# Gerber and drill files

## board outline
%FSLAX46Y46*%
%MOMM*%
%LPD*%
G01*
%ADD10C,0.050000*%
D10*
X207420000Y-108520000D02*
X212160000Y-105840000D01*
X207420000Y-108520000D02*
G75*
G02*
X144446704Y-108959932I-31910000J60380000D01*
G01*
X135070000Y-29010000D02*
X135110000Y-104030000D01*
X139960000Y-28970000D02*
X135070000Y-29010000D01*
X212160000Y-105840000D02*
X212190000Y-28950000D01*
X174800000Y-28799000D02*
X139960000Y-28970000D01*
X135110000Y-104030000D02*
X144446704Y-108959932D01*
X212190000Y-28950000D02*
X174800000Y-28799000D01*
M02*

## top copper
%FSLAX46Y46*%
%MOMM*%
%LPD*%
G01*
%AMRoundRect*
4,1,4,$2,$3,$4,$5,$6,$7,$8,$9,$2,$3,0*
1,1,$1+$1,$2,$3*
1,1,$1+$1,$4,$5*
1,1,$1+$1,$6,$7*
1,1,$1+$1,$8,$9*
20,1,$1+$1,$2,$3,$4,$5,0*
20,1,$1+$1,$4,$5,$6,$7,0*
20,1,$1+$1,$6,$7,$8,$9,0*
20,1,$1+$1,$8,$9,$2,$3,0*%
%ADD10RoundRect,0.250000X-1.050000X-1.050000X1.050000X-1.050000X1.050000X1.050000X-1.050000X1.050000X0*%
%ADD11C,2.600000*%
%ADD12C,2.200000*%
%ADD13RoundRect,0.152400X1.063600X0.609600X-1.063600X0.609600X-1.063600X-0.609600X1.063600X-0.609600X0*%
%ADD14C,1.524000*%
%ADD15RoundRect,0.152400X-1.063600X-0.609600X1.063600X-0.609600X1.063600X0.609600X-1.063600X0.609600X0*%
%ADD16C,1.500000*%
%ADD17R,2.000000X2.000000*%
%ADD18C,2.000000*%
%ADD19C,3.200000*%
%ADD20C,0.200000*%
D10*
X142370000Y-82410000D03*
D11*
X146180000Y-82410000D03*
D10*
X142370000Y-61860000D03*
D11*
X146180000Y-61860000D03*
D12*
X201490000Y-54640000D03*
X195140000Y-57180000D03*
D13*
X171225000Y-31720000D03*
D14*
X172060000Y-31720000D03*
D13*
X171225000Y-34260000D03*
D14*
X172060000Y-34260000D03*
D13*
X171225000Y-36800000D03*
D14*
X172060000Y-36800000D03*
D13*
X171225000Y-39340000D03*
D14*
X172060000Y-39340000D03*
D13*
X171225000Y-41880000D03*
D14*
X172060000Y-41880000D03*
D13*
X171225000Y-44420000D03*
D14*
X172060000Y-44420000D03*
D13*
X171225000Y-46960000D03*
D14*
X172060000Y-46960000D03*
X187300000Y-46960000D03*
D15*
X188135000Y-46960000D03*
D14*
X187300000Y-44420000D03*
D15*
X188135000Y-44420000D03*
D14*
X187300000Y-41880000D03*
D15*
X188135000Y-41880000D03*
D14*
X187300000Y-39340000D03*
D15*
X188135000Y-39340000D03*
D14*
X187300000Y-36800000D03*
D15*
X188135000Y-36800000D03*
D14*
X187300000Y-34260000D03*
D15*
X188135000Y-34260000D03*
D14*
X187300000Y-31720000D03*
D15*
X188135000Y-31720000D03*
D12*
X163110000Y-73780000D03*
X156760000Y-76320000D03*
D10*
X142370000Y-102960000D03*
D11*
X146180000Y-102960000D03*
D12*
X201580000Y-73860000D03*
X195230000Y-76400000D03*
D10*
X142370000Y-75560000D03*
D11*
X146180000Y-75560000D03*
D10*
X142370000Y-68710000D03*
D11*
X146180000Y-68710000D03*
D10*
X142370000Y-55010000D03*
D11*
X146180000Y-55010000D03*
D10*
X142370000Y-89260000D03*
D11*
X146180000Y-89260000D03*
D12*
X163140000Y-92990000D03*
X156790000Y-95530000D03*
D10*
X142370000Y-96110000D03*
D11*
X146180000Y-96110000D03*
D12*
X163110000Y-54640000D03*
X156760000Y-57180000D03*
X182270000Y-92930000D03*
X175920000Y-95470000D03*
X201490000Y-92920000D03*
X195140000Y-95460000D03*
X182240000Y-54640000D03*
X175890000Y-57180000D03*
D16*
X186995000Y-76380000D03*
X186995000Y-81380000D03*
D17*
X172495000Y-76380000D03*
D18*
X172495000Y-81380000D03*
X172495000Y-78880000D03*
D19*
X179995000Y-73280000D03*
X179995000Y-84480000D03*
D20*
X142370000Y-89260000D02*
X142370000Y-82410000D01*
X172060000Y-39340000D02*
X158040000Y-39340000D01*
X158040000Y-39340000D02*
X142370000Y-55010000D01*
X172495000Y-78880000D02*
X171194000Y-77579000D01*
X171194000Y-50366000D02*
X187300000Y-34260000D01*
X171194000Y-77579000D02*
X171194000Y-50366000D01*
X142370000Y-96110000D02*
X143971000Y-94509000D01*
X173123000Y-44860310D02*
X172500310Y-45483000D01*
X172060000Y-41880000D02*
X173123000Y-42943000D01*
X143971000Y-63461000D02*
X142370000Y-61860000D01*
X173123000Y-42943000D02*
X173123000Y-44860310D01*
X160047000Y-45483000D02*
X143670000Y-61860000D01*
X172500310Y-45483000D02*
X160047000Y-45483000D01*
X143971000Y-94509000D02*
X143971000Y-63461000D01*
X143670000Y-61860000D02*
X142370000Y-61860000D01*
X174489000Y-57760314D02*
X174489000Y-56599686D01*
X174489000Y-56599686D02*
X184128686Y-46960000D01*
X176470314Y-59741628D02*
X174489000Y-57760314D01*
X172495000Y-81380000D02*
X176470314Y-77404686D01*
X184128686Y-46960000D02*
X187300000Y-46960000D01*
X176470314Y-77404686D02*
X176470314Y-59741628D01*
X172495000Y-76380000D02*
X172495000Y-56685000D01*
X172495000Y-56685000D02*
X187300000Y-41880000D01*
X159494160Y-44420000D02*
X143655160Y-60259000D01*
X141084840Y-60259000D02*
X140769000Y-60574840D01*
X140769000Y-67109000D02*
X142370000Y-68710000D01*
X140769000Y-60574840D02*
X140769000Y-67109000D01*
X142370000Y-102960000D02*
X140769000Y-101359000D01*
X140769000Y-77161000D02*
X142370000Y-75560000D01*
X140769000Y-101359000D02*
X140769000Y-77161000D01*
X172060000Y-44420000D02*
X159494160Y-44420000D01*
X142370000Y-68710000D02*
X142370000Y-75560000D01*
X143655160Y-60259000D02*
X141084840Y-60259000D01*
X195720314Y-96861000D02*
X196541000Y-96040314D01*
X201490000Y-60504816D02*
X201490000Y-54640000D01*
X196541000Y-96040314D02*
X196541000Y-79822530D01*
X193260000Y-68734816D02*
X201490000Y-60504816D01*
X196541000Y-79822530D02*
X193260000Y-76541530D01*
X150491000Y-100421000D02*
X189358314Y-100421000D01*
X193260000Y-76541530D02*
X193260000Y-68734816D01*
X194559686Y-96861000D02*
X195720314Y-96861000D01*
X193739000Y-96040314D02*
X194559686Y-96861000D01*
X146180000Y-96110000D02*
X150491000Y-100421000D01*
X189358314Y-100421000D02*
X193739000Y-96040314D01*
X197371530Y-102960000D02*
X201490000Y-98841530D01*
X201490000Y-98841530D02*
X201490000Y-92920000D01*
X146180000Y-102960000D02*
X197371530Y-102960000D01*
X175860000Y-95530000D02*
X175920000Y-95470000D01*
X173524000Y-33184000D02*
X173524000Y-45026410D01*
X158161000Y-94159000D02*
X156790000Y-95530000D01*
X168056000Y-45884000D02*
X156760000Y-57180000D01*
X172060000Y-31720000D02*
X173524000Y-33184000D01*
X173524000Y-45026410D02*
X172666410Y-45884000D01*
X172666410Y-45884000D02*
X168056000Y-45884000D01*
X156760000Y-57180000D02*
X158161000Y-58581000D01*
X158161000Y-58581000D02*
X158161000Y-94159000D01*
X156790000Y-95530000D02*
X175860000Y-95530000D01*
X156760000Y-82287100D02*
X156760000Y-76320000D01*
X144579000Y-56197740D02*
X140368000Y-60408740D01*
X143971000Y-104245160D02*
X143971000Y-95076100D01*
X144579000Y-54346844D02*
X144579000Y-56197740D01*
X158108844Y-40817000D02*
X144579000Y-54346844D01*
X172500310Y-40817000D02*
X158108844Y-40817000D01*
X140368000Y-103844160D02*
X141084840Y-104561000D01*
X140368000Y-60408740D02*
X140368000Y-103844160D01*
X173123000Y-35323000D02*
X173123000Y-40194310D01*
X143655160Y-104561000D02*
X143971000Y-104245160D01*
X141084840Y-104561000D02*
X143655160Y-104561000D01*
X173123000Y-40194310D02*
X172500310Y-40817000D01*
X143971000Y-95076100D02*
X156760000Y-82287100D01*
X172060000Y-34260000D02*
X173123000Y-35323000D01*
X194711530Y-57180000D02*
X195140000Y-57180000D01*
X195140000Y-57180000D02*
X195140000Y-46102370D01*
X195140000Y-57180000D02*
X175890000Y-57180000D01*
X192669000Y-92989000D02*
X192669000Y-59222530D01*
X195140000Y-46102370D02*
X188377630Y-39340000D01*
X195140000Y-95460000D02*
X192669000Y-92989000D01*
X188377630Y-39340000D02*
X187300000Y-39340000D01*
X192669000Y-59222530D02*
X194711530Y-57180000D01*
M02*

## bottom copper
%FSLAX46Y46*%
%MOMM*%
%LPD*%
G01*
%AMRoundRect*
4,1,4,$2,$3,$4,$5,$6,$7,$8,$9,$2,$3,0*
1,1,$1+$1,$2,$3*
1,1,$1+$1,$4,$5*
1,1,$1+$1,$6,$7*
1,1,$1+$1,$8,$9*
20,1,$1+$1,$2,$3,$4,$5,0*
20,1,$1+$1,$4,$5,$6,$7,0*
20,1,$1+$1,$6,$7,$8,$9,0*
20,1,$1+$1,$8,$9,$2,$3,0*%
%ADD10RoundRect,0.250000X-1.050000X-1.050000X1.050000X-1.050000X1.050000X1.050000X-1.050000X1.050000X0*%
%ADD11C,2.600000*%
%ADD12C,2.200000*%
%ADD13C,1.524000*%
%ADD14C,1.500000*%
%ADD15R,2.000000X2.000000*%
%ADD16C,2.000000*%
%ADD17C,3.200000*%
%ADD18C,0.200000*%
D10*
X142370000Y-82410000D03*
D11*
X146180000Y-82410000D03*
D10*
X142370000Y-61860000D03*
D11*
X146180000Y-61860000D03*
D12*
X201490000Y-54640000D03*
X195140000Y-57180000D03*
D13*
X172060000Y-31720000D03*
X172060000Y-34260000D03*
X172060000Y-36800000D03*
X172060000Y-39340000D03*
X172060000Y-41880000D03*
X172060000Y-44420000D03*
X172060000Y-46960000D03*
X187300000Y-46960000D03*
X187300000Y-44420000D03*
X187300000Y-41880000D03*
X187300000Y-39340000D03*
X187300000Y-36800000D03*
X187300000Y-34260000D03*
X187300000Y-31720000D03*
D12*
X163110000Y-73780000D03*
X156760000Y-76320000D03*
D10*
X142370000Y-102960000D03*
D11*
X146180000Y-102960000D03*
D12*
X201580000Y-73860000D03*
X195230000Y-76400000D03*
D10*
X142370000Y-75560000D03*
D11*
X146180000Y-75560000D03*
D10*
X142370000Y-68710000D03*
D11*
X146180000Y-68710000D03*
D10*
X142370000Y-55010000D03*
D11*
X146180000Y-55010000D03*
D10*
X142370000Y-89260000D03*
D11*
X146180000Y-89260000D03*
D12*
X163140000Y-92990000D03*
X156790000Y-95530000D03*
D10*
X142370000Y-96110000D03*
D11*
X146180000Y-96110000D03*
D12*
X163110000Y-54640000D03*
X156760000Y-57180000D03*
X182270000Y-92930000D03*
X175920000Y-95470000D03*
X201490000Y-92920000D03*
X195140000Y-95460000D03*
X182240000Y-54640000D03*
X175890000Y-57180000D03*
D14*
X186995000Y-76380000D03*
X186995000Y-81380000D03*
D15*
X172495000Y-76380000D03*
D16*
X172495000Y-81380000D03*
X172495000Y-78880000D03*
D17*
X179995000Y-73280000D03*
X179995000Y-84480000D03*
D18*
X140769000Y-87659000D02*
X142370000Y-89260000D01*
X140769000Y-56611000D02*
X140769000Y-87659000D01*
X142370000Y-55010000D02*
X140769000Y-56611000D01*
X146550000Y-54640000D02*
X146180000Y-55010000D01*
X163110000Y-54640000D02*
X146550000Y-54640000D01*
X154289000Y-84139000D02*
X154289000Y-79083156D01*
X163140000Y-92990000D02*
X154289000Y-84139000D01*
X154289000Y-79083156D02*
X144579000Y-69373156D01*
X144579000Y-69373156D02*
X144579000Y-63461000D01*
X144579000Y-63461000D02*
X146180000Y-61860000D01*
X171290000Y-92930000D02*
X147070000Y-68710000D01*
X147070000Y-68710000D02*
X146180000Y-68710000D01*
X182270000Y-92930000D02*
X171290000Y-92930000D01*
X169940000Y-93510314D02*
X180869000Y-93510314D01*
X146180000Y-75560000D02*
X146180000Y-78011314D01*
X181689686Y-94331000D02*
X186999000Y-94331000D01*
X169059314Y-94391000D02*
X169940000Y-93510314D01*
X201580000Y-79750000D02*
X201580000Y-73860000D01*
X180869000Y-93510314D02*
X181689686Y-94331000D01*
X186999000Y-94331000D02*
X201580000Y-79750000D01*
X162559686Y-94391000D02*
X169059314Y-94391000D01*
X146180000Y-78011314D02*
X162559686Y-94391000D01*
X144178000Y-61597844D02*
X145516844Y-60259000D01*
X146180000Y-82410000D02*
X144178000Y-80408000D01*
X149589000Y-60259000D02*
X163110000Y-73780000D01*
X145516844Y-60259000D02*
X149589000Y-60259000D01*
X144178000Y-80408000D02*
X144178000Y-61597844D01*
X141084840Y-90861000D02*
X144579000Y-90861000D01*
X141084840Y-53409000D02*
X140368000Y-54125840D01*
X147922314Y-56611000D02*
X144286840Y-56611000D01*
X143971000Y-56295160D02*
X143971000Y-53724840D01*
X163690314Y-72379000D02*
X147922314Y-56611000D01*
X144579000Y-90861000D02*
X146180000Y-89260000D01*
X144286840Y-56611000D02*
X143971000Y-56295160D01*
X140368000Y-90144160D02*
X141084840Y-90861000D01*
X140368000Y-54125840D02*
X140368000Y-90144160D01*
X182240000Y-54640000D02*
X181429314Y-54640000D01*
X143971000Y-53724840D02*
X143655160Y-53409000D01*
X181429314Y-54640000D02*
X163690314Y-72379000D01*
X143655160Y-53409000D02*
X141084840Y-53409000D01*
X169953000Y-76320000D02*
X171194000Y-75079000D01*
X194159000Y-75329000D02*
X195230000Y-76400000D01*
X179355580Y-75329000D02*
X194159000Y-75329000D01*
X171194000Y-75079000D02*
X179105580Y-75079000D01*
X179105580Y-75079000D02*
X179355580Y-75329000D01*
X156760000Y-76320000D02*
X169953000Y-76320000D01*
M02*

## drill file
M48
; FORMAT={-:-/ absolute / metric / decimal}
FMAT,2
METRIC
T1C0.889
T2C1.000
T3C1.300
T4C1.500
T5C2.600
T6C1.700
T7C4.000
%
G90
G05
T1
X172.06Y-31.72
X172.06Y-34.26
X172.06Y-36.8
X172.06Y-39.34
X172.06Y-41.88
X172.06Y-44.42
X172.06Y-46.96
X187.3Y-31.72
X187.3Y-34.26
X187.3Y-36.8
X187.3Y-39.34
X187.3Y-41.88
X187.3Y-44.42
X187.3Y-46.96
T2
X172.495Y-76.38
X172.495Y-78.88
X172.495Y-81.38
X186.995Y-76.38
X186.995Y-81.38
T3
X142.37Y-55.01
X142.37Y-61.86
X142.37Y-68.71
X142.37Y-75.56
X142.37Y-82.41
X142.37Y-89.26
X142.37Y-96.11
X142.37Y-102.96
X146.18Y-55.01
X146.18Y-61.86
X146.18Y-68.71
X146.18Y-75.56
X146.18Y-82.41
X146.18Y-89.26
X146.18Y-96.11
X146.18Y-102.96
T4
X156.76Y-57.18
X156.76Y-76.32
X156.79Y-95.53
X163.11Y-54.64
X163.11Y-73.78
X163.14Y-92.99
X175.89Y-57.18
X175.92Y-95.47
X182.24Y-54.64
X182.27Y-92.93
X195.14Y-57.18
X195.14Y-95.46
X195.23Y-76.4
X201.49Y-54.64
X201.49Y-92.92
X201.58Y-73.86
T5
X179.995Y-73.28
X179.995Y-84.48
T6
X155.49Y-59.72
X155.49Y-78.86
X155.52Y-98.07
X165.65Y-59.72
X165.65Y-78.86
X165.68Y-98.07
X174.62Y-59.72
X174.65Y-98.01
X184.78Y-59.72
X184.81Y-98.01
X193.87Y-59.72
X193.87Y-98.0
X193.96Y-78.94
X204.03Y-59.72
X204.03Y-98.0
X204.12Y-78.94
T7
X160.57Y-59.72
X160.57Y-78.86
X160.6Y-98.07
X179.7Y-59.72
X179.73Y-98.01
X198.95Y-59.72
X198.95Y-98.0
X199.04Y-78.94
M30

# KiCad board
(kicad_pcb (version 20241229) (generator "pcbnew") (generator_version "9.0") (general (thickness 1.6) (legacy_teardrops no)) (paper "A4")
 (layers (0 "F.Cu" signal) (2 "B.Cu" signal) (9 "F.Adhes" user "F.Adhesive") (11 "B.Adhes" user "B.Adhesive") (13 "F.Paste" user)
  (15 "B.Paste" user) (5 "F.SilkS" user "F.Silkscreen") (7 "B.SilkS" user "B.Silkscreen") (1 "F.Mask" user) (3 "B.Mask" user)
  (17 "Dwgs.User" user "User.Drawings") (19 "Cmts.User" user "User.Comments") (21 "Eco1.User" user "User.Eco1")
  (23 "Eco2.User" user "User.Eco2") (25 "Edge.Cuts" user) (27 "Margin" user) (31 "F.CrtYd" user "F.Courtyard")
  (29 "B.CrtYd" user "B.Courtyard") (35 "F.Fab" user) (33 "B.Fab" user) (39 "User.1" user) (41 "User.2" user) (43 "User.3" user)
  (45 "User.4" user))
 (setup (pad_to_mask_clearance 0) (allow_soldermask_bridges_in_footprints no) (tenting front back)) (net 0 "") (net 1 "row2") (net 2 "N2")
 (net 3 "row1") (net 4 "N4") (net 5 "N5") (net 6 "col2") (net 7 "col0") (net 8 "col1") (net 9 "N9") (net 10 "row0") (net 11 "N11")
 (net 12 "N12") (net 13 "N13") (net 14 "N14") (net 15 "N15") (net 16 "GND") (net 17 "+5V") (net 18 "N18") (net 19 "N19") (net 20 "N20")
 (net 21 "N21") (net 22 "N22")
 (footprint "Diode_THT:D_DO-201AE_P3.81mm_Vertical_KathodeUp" (layer "F.Cu") (at 142.37 82.41)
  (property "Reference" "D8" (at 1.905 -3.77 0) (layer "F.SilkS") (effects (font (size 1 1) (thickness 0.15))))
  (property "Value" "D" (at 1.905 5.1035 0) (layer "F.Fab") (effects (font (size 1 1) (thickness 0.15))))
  (pad "1" thru_hole roundrect (at 0 0) (size 2.6 2.6) (drill 1.3) (layers "*.Cu" "*.Mask") (remove_unused_layers no)
   (roundrect_rratio 0.096154) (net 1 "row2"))
  (pad "2" thru_hole circle (at 3.81 0) (size 2.6 2.6) (drill 1.3) (layers "*.Cu" "*.Mask") (remove_unused_layers no) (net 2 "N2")))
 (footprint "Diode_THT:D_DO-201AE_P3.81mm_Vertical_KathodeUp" (layer "F.Cu") (at 142.37 61.86)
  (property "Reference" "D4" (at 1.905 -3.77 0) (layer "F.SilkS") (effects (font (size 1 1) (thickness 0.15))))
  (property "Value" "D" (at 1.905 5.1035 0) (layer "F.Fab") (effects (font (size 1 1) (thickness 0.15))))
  (pad "1" thru_hole roundrect (at 0 0) (size 2.6 2.6) (drill 1.3) (layers "*.Cu" "*.Mask") (remove_unused_layers no)
   (roundrect_rratio 0.096154) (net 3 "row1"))
  (pad "2" thru_hole circle (at 3.81 0) (size 2.6 2.6) (drill 1.3) (layers "*.Cu" "*.Mask") (remove_unused_layers no) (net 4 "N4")))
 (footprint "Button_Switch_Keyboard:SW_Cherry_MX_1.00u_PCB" (layer "F.Cu") (at 201.49 54.64)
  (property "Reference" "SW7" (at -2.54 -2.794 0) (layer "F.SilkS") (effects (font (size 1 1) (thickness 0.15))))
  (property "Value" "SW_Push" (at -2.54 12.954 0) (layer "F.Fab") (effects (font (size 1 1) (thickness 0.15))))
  (pad "" np_thru_hole circle (at -7.62 5.08) (size 1.7 1.7) (drill 1.7) (layers "*.Cu" "*.Mask"))
  (pad "" np_thru_hole circle (at -2.54 5.08) (size 4 4) (drill 4) (layers "*.Cu" "*.Mask"))
  (pad "" np_thru_hole circle (at 2.54 5.08) (size 1.7 1.7) (drill 1.7) (layers "*.Cu" "*.Mask"))
  (pad "1" thru_hole circle (at 0 0) (size 2.2 2.2) (drill 1.5) (layers "*.Cu" "*.Mask") (remove_unused_layers no) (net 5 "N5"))
  (pad "2" thru_hole circle (at -6.35 2.54) (size 2.2 2.2) (drill 1.5) (layers "*.Cu" "*.Mask") (remove_unused_layers no) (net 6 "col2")))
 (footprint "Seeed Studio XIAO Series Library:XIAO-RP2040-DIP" (layer "F.Cu") (at 179.68 39.34)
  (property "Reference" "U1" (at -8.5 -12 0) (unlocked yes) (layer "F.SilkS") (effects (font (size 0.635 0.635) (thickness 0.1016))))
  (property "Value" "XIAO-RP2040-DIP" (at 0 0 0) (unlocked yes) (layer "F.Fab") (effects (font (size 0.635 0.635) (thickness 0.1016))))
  (pad "1" smd roundrect (at -8.455 -7.62 180) (size 2.432 1.524) (layers "F.Cu" "F.Mask") (roundrect_rratio 0.1) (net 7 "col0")
   (thermal_bridge_angle 45))
  (pad "1" thru_hole circle (at -7.62 -7.62 180) (size 1.524 1.524) (drill 0.889) (layers "*.Cu" "*.Mask") (remove_unused_layers no)
   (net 7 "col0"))
  (pad "2" smd roundrect (at -8.455 -5.08 180) (size 2.432 1.524) (layers "F.Cu" "F.Mask") (roundrect_rratio 0.1) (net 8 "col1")
   (thermal_bridge_angle 45))
  (pad "2" thru_hole circle (at -7.62 -5.08 180) (size 1.524 1.524) (drill 0.889) (layers "*.Cu" "*.Mask") (remove_unused_layers no)
   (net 8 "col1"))
  (pad "3" smd roundrect (at -8.455 -2.54 180) (size 2.432 1.524) (layers "F.Cu" "F.Mask") (roundrect_rratio 0.1) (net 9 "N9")
   (thermal_bridge_angle 45))
  (pad "3" thru_hole circle (at -7.62 -2.54 180) (size 1.524 1.524) (drill 0.889) (layers "*.Cu" "*.Mask") (remove_unused_layers no)
   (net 9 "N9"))
  (pad "4" smd roundrect (at -8.455 0 180) (size 2.432 1.524) (layers "F.Cu" "F.Mask") (roundrect_rratio 0.1) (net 1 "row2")
   (thermal_bridge_angle 45))
  (pad "4" thru_hole circle (at -7.62 0 180) (size 1.524 1.524) (drill 0.889) (layers "*.Cu" "*.Mask") (remove_unused_layers no)
   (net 1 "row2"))
  (pad "5" smd roundrect (at -8.455 2.54 180) (size 2.432 1.524) (layers "F.Cu" "F.Mask") (roundrect_rratio 0.1) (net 3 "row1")
   (thermal_bridge_angle 45))
  (pad "5" thru_hole circle (at -7.62 2.54 180) (size 1.524 1.524) (drill 0.889) (layers "*.Cu" "*.Mask") (remove_unused_layers no)
   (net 3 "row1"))
  (pad "6" smd roundrect (at -8.455 5.08 180) (size 2.432 1.524) (layers "F.Cu" "F.Mask") (roundrect_rratio 0.1) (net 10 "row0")
   (thermal_bridge_angle 45))
  (pad "6" thru_hole circle (at -7.62 5.08 180) (size 1.524 1.524) (drill 0.889) (layers "*.Cu" "*.Mask") (remove_unused_layers no)
   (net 10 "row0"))
  (pad "7" smd roundrect (at -8.455 7.62 180) (size 2.432 1.524) (layers "F.Cu" "F.Mask") (roundrect_rratio 0.1) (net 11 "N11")
   (thermal_bridge_angle 45))
  (pad "7" thru_hole circle (at -7.62 7.62 180) (size 1.524 1.524) (drill 0.889) (layers "*.Cu" "*.Mask") (remove_unused_layers no)
   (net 11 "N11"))
  (pad "8" thru_hole circle (at 7.62 7.62) (size 1.524 1.524) (drill 0.889) (layers "*.Cu" "*.Mask") (remove_unused_layers no)
   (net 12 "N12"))
  (pad "8" smd roundrect (at 8.455 7.62) (size 2.432 1.524) (layers "F.Cu" "F.Mask") (roundrect_rratio 0.1) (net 12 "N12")
   (thermal_bridge_angle 45))
  (pad "9" thru_hole circle (at 7.62 5.08) (size 1.524 1.524) (drill 0.889) (layers "*.Cu" "*.Mask") (remove_unused_layers no)
   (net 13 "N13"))
  (pad "9" smd roundrect (at 8.455 5.08) (size 2.432 1.524) (layers "F.Cu" "F.Mask") (roundrect_rratio 0.1) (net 13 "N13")
   (thermal_bridge_angle 45))
  (pad "10" thru_hole circle (at 7.62 2.54) (size 1.524 1.524) (drill 0.889) (layers "*.Cu" "*.Mask") (remove_unused_layers no)
   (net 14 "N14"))
  (pad "10" smd roundrect (at 8.455 2.54) (size 2.432 1.524) (layers "F.Cu" "F.Mask") (roundrect_rratio 0.1) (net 14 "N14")
   (thermal_bridge_angle 45))
  (pad "11" thru_hole circle (at 7.62 0) (size 1.524 1.524) (drill 0.889) (layers "*.Cu" "*.Mask") (remove_unused_layers no) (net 6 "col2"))
  (pad "11" smd roundrect (at 8.455 0) (size 2.432 1.524) (layers "F.Cu" "F.Mask") (roundrect_rratio 0.1) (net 6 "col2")
   (thermal_bridge_angle 45))
  (pad "12" thru_hole circle (at 7.62 -2.54) (size 1.524 1.524) (drill 0.889) (layers "*.Cu" "*.Mask") (remove_unused_layers no)
   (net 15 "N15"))
  (pad "12" smd roundrect (at 8.455 -2.54) (size 2.432 1.524) (layers "F.Cu" "F.Mask") (roundrect_rratio 0.1) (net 15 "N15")
   (thermal_bridge_angle 45))
  (pad "13" thru_hole circle (at 7.62 -5.08) (size 1.524 1.524) (drill 0.889) (layers "*.Cu" "*.Mask") (remove_unused_layers no)
   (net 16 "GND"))
  (pad "13" smd roundrect (at 8.455 -5.08) (size 2.432 1.524) (layers "F.Cu" "F.Mask") (roundrect_rratio 0.1) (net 16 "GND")
   (thermal_bridge_angle 45))
  (pad "14" thru_hole circle (at 7.62 -7.62) (size 1.524 1.524) (drill 0.889) (layers "*.Cu" "*.Mask") (remove_unused_layers no)
   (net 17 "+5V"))
  (pad "14" smd roundrect (at 8.455 -7.62) (size 2.432 1.524) (layers "F.Cu" "F.Mask") (roundrect_rratio 0.1) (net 17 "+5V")
   (thermal_bridge_angle 45)))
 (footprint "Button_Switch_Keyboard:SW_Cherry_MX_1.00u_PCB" (layer "F.Cu") (at 163.11 73.78)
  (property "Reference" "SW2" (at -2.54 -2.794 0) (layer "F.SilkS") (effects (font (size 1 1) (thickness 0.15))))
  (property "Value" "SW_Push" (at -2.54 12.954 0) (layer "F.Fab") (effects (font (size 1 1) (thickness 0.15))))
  (pad "" np_thru_hole circle (at -7.62 5.08) (size 1.7 1.7) (drill 1.7) (layers "*.Cu" "*.Mask"))
  (pad "" np_thru_hole circle (at -2.54 5.08) (size 4 4) (drill 4) (layers "*.Cu" "*.Mask"))
  (pad "" np_thru_hole circle (at 2.54 5.08) (size 1.7 1.7) (drill 1.7) (layers "*.Cu" "*.Mask"))
  (pad "1" thru_hole circle (at 0 0) (size 2.2 2.2) (drill 1.5) (layers "*.Cu" "*.Mask") (remove_unused_layers no) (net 2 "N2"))
  (pad "2" thru_hole circle (at -6.35 2.54) (size 2.2 2.2) (drill 1.5) (layers "*.Cu" "*.Mask") (remove_unused_layers no) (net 8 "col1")))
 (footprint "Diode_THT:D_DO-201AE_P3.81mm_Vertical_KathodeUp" (layer "F.Cu") (at 142.37 102.96)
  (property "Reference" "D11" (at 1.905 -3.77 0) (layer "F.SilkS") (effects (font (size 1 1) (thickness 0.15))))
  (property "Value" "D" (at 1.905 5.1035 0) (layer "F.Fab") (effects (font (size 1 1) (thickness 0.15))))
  (pad "1" thru_hole roundrect (at 0 0) (size 2.6 2.6) (drill 1.3) (layers "*.Cu" "*.Mask") (remove_unused_layers no)
   (roundrect_rratio 0.096154) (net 10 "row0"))
  (pad "2" thru_hole circle (at 3.81 0) (size 2.6 2.6) (drill 1.3) (layers "*.Cu" "*.Mask") (remove_unused_layers no) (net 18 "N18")))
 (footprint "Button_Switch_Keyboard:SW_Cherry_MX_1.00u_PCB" (layer "F.Cu") (at 201.58 73.86)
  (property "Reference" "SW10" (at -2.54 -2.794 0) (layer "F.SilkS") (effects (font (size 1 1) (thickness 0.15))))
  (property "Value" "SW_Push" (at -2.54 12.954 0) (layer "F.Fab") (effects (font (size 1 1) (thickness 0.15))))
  (pad "" np_thru_hole circle (at -7.62 5.08) (size 1.7 1.7) (drill 1.7) (layers "*.Cu" "*.Mask"))
  (pad "" np_thru_hole circle (at -2.54 5.08) (size 4 4) (drill 4) (layers "*.Cu" "*.Mask"))
  (pad "" np_thru_hole circle (at 2.54 5.08) (size 1.7 1.7) (drill 1.7) (layers "*.Cu" "*.Mask"))
  (pad "1" thru_hole circle (at 0 0) (size 2.2 2.2) (drill 1.5) (layers "*.Cu" "*.Mask") (remove_unused_layers no) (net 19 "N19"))
  (pad "2" thru_hole circle (at -6.35 2.54) (size 2.2 2.2) (drill 1.5) (layers "*.Cu" "*.Mask") (remove_unused_layers no) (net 8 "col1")))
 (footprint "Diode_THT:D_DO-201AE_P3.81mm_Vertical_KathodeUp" (layer "F.Cu") (at 142.37 75.56)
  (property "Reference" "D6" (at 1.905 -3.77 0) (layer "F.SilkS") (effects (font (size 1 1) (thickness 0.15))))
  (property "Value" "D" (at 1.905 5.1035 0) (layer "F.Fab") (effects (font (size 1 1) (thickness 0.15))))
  (pad "1" thru_hole roundrect (at 0 0) (size 2.6 2.6) (drill 1.3) (layers "*.Cu" "*.Mask") (remove_unused_layers no)
   (roundrect_rratio 0.096154) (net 10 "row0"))
  (pad "2" thru_hole circle (at 3.81 0) (size 2.6 2.6) (drill 1.3) (layers "*.Cu" "*.Mask") (remove_unused_layers no) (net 19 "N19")))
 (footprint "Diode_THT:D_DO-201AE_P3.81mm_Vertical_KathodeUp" (layer "F.Cu") (at 142.37 68.71)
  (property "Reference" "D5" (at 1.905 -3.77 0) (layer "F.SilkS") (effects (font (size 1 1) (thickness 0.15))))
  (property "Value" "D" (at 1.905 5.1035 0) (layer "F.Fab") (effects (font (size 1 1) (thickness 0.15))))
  (pad "1" thru_hole roundrect (at 0 0) (size 2.6 2.6) (drill 1.3) (layers "*.Cu" "*.Mask") (remove_unused_layers no)
   (roundrect_rratio 0.096154) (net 10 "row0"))
  (pad "2" thru_hole circle (at 3.81 0) (size 2.6 2.6) (drill 1.3) (layers "*.Cu" "*.Mask") (remove_unused_layers no) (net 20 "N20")))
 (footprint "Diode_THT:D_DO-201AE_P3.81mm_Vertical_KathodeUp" (layer "F.Cu") (at 142.37 55.01)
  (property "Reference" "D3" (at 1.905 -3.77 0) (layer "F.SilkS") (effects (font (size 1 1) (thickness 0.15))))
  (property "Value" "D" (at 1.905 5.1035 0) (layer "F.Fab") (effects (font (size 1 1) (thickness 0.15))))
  (pad "1" thru_hole roundrect (at 0 0) (size 2.6 2.6) (drill 1.3) (layers "*.Cu" "*.Mask") (remove_unused_layers no)
   (roundrect_rratio 0.096154) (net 1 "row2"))
  (pad "2" thru_hole circle (at 3.81 0) (size 2.6 2.6) (drill 1.3) (layers "*.Cu" "*.Mask") (remove_unused_layers no) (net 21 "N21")))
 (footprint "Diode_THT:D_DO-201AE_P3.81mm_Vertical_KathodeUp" (layer "F.Cu") (at 142.37 89.26)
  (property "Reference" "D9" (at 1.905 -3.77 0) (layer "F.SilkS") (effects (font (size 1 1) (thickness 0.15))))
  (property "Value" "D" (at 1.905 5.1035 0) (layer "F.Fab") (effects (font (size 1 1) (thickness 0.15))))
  (pad "1" thru_hole roundrect (at 0 0) (size 2.6 2.6) (drill 1.3) (layers "*.Cu" "*.Mask") (remove_unused_layers no)
   (roundrect_rratio 0.096154) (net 1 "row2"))
  (pad "2" thru_hole circle (at 3.81 0) (size 2.6 2.6) (drill 1.3) (layers "*.Cu" "*.Mask") (remove_unused_layers no) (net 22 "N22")))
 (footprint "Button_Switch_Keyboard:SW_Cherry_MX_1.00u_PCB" (layer "F.Cu") (at 163.14 92.99)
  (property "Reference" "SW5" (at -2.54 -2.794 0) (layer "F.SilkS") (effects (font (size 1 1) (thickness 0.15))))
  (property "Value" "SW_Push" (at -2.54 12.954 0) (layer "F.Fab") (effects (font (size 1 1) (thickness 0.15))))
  (pad "" np_thru_hole circle (at -7.62 5.08) (size 1.7 1.7) (drill 1.7) (layers "*.Cu" "*.Mask"))
  (pad "" np_thru_hole circle (at -2.54 5.08) (size 4 4) (drill 4) (layers "*.Cu" "*.Mask"))
  (pad "" np_thru_hole circle (at 2.54 5.08) (size 1.7 1.7) (drill 1.7) (layers "*.Cu" "*.Mask"))
  (pad "1" thru_hole circle (at 0 0) (size 2.2 2.2) (drill 1.5) (layers "*.Cu" "*.Mask") (remove_unused_layers no) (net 4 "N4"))
  (pad "2" thru_hole circle (at -6.35 2.54) (size 2.2 2.2) (drill 1.5) (layers "*.Cu" "*.Mask") (remove_unused_layers no) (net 7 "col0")))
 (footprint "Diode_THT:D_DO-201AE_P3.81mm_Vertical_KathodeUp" (layer "F.Cu") (at 142.37 96.11)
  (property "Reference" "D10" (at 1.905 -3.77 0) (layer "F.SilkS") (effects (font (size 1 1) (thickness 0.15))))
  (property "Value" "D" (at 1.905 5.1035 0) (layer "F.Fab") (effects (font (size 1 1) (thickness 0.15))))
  (pad "1" thru_hole roundrect (at 0 0) (size 2.6 2.6) (drill 1.3) (layers "*.Cu" "*.Mask") (remove_unused_layers no)
   (roundrect_rratio 0.096154) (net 3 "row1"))
  (pad "2" thru_hole circle (at 3.81 0) (size 2.6 2.6) (drill 1.3) (layers "*.Cu" "*.Mask") (remove_unused_layers no) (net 5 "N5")))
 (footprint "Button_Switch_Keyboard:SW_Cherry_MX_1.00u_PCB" (layer "F.Cu") (at 163.11 54.64)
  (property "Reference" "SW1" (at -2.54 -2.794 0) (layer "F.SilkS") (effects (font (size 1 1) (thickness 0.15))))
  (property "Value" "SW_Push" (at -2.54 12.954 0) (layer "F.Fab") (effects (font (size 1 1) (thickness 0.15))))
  (pad "" np_thru_hole circle (at -7.62 5.08) (size 1.7 1.7) (drill 1.7) (layers "*.Cu" "*.Mask"))
  (pad "" np_thru_hole circle (at -2.54 5.08) (size 4 4) (drill 4) (layers "*.Cu" "*.Mask"))
  (pad "" np_thru_hole circle (at 2.54 5.08) (size 1.7 1.7) (drill 1.7) (layers "*.Cu" "*.Mask"))
  (pad "1" thru_hole circle (at 0 0) (size 2.2 2.2) (drill 1.5) (layers "*.Cu" "*.Mask") (remove_unused_layers no) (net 21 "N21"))
  (pad "2" thru_hole circle (at -6.35 2.54) (size 2.2 2.2) (drill 1.5) (layers "*.Cu" "*.Mask") (remove_unused_layers no) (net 7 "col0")))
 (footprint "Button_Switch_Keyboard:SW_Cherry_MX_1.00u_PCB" (layer "F.Cu") (at 182.27 92.93)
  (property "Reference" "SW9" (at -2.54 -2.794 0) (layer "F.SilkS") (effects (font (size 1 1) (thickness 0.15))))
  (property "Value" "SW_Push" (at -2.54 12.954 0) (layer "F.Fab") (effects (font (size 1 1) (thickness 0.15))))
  (pad "" np_thru_hole circle (at -7.62 5.08) (size 1.7 1.7) (drill 1.7) (layers "*.Cu" "*.Mask"))
  (pad "" np_thru_hole circle (at -2.54 5.08) (size 4 4) (drill 4) (layers "*.Cu" "*.Mask"))
  (pad "" np_thru_hole circle (at 2.54 5.08) (size 1.7 1.7) (drill 1.7) (layers "*.Cu" "*.Mask"))
  (pad "1" thru_hole circle (at 0 0) (size 2.2 2.2) (drill 1.5) (layers "*.Cu" "*.Mask") (remove_unused_layers no) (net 20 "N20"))
  (pad "2" thru_hole circle (at -6.35 2.54) (size 2.2 2.2) (drill 1.5) (layers "*.Cu" "*.Mask") (remove_unused_layers no) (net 7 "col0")))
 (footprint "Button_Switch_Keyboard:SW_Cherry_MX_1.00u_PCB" (layer "F.Cu") (at 201.49 92.92)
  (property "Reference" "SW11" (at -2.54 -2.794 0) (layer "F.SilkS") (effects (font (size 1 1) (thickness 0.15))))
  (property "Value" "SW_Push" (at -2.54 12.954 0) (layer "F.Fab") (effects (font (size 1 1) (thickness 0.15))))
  (pad "" np_thru_hole circle (at -7.62 5.08) (size 1.7 1.7) (drill 1.7) (layers "*.Cu" "*.Mask"))
  (pad "" np_thru_hole circle (at -2.54 5.08) (size 4 4) (drill 4) (layers "*.Cu" "*.Mask"))
  (pad "" np_thru_hole circle (at 2.54 5.08) (size 1.7 1.7) (drill 1.7) (layers "*.Cu" "*.Mask"))
  (pad "1" thru_hole circle (at 0 0) (size 2.2 2.2) (drill 1.5) (layers "*.Cu" "*.Mask") (remove_unused_layers no) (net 18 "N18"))
  (pad "2" thru_hole circle (at -6.35 2.54) (size 2.2 2.2) (drill 1.5) (layers "*.Cu" "*.Mask") (remove_unused_layers no) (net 6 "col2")))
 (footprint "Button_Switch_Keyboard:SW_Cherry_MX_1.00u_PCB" (layer "F.Cu") (at 182.24 54.64)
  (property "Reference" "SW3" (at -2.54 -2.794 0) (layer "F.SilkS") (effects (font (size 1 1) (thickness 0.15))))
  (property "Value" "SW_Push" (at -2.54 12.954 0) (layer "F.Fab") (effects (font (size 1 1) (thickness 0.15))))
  (pad "" np_thru_hole circle (at -7.62 5.08) (size 1.7 1.7) (drill 1.7) (layers "*.Cu" "*.Mask"))
  (pad "" np_thru_hole circle (at -2.54 5.08) (size 4 4) (drill 4) (layers "*.Cu" "*.Mask"))
  (pad "" np_thru_hole circle (at 2.54 5.08) (size 1.7 1.7) (drill 1.7) (layers "*.Cu" "*.Mask"))
  (pad "1" thru_hole circle (at 0 0) (size 2.2 2.2) (drill 1.5) (layers "*.Cu" "*.Mask") (remove_unused_layers no) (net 22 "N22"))
  (pad "2" thru_hole circle (at -6.35 2.54) (size 2.2 2.2) (drill 1.5) (layers "*.Cu" "*.Mask") (remove_unused_layers no) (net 6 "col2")))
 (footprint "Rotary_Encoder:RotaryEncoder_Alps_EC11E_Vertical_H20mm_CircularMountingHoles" (layer "F.Cu") (at 172.495 76.38)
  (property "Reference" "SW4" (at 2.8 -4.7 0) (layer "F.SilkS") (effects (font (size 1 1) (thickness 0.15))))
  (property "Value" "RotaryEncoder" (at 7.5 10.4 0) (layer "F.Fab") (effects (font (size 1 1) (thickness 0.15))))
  (pad "" thru_hole circle (at 14.5 0) (size 1.5 1.5) (drill 1) (layers "*.Cu" "*.Mask") (remove_unused_layers no))
  (pad "" thru_hole circle (at 14.5 5) (size 1.5 1.5) (drill 1) (layers "*.Cu" "*.Mask") (remove_unused_layers no))
  (pad "A" thru_hole rect (at 0 0) (size 2 2) (drill 1) (layers "*.Cu" "*.Mask") (remove_unused_layers no) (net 14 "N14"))
  (pad "B" thru_hole circle (at 0 5) (size 2 2) (drill 1) (layers "*.Cu" "*.Mask") (remove_unused_layers no) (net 12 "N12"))
  (pad "C" thru_hole circle (at 0 2.5) (size 2 2) (drill 1) (layers "*.Cu" "*.Mask") (remove_unused_layers no) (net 16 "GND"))
  (pad "MP" thru_hole circle (at 7.5 -3.1) (size 3.2 3.2) (drill 2.6) (layers "*.Cu" "*.Mask") (remove_unused_layers no))
  (pad "MP" thru_hole circle (at 7.5 8.1) (size 3.2 3.2) (drill 2.6) (layers "*.Cu" "*.Mask") (remove_unused_layers no)))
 (gr_line (start 207.42 108.52) (end 212.16 105.84) (stroke (width 0.05) (type default)) (layer "Edge.Cuts"))
 (gr_arc (start 207.42 108.52) (mid 175.987087 116.431763) (end 144.446704 108.959932) (stroke (width 0.05) (type default))
  (layer "Edge.Cuts"))
 (gr_line (start 135.07 29.01) (end 135.11 104.03) (stroke (width 0.05) (type default)) (layer "Edge.Cuts"))
 (gr_line (start 139.96 28.97) (end 135.07 29.01) (stroke (width 0.05) (type default)) (layer "Edge.Cuts"))
 (gr_line (start 212.16 105.84) (end 212.19 28.95) (stroke (width 0.05) (type default)) (layer "Edge.Cuts"))
 (gr_line (start 174.8 28.799) (end 139.96 28.97) (stroke (width 0.05) (type default)) (layer "Edge.Cuts"))
 (gr_line (start 135.11 104.03) (end 144.446704 108.959932) (stroke (width 0.05) (type default)) (layer "Edge.Cuts"))
 (gr_line (start 212.19 28.95) (end 174.8 28.799) (stroke (width 0.05) (type default)) (layer "Edge.Cuts"))
 (segment (start 142.37 89.26) (end 142.37 82.41) (width 0.2) (layer "F.Cu") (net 1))
 (segment (start 172.06 39.34) (end 158.04 39.34) (width 0.2) (layer "F.Cu") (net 1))
 (segment (start 158.04 39.34) (end 142.37 55.01) (width 0.2) (layer "F.Cu") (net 1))
 (segment (start 140.769 87.659) (end 142.37 89.26) (width 0.2) (layer "B.Cu") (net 1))
 (segment (start 140.769 56.611) (end 140.769 87.659) (width 0.2) (layer "B.Cu") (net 1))
 (segment (start 142.37 55.01) (end 140.769 56.611) (width 0.2) (layer "B.Cu") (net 1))
 (segment (start 172.495 78.88) (end 171.194 77.579) (width 0.2) (layer "F.Cu") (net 16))
 (segment (start 171.194 50.366) (end 187.3 34.26) (width 0.2) (layer "F.Cu") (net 16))
 (segment (start 171.194 77.579) (end 171.194 50.366) (width 0.2) (layer "F.Cu") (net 16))
 (segment (start 146.55 54.64) (end 146.18 55.01) (width 0.2) (layer "B.Cu") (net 21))
 (segment (start 163.11 54.64) (end 146.55 54.64) (width 0.2) (layer "B.Cu") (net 21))
 (segment (start 142.37 96.11) (end 143.971 94.509) (width 0.2) (layer "F.Cu") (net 3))
 (segment (start 173.123 44.86031) (end 172.50031 45.483) (width 0.2) (layer "F.Cu") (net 3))
 (segment (start 172.06 41.88) (end 173.123 42.943) (width 0.2) (layer "F.Cu") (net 3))
 (segment (start 143.971 63.461) (end 142.37 61.86) (width 0.2) (layer "F.Cu") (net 3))
 (segment (start 173.123 42.943) (end 173.123 44.86031) (width 0.2) (layer "F.Cu") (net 3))
 (segment (start 160.047 45.483) (end 143.67 61.86) (width 0.2) (layer "F.Cu") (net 3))
 (segment (start 172.50031 45.483) (end 160.047 45.483) (width 0.2) (layer "F.Cu") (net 3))
 (segment (start 143.971 94.509) (end 143.971 63.461) (width 0.2) (layer "F.Cu") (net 3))
 (segment (start 143.67 61.86) (end 142.37 61.86) (width 0.2) (layer "F.Cu") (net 3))
 (segment (start 174.489 57.760314) (end 174.489 56.599686) (width 0.2) (layer "F.Cu") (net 12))
 (segment (start 174.489 56.599686) (end 184.128686 46.96) (width 0.2) (layer "F.Cu") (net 12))
 (segment (start 176.470314 59.741628) (end 174.489 57.760314) (width 0.2) (layer "F.Cu") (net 12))
 (segment (start 172.495 81.38) (end 176.470314 77.404686) (width 0.2) (layer "F.Cu") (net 12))
 (segment (start 184.128686 46.96) (end 187.3 46.96) (width 0.2) (layer "F.Cu") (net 12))
 (segment (start 176.470314 77.404686) (end 176.470314 59.741628) (width 0.2) (layer "F.Cu") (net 12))
 (segment (start 154.289 84.139) (end 154.289 79.083156) (width 0.2) (layer "B.Cu") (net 4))
 (segment (start 163.14 92.99) (end 154.289 84.139) (width 0.2) (layer "B.Cu") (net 4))
 (segment (start 154.289 79.083156) (end 144.579 69.373156) (width 0.2) (layer "B.Cu") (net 4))
 (segment (start 144.579 69.373156) (end 144.579 63.461) (width 0.2) (layer "B.Cu") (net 4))
 (segment (start 144.579 63.461) (end 146.18 61.86) (width 0.2) (layer "B.Cu") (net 4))
 (segment (start 172.495 76.38) (end 172.495 56.685) (width 0.2) (layer "F.Cu") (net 14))
 (segment (start 172.495 56.685) (end 187.3 41.88) (width 0.2) (layer "F.Cu") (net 14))
 (segment (start 159.49416 44.42) (end 143.65516 60.259) (width 0.2) (layer "F.Cu") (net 10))
 (segment (start 141.08484 60.259) (end 140.769 60.57484) (width 0.2) (layer "F.Cu") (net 10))
 (segment (start 140.769 67.109) (end 142.37 68.71) (width 0.2) (layer "F.Cu") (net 10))
 (segment (start 140.769 60.57484) (end 140.769 67.109) (width 0.2) (layer "F.Cu") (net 10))
 (segment (start 142.37 102.96) (end 140.769 101.359) (width 0.2) (layer "F.Cu") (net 10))
 (segment (start 140.769 77.161) (end 142.37 75.56) (width 0.2) (layer "F.Cu") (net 10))
 (segment (start 140.769 101.359) (end 140.769 77.161) (width 0.2) (layer "F.Cu") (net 10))
 (segment (start 172.06 44.42) (end 159.49416 44.42) (width 0.2) (layer "F.Cu") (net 10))
 (segment (start 142.37 68.71) (end 142.37 75.56) (width 0.2) (layer "F.Cu") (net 10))
 (segment (start 143.65516 60.259) (end 141.08484 60.259) (width 0.2) (layer "F.Cu") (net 10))
 (segment (start 171.29 92.93) (end 147.07 68.71) (width 0.2) (layer "B.Cu") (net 20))
 (segment (start 147.07 68.71) (end 146.18 68.71) (width 0.2) (layer "B.Cu") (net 20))
 (segment (start 182.27 92.93) (end 171.29 92.93) (width 0.2) (layer "B.Cu") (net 20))
 (segment (start 169.94 93.510314) (end 180.869 93.510314) (width 0.2) (layer "B.Cu") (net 19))
 (segment (start 146.18 75.56) (end 146.18 78.011314) (width 0.2) (layer "B.Cu") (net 19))
 (segment (start 181.689686 94.331) (end 186.999 94.331) (width 0.2) (layer "B.Cu") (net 19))
 (segment (start 169.059314 94.391) (end 169.94 93.510314) (width 0.2) (layer "B.Cu") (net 19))
 (segment (start 201.58 79.75) (end 201.58 73.86) (width 0.2) (layer "B.Cu") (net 19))
 (segment (start 180.869 93.510314) (end 181.689686 94.331) (width 0.2) (layer "B.Cu") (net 19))
 (segment (start 186.999 94.331) (end 201.58 79.75) (width 0.2) (layer "B.Cu") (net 19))
 (segment (start 162.559686 94.391) (end 169.059314 94.391) (width 0.2) (layer "B.Cu") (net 19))
 (segment (start 146.18 78.011314) (end 162.559686 94.391) (width 0.2) (layer "B.Cu") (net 19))
 (segment (start 144.178 61.597844) (end 145.516844 60.259) (width 0.2) (layer "B.Cu") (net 2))
 (segment (start 146.18 82.41) (end 144.178 80.408) (width 0.2) (layer "B.Cu") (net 2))
 (segment (start 149.589 60.259) (end 163.11 73.78) (width 0.2) (layer "B.Cu") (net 2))
 (segment (start 145.516844 60.259) (end 149.589 60.259) (width 0.2) (layer "B.Cu") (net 2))
 (segment (start 144.178 80.408) (end 144.178 61.597844) (width 0.2) (layer "B.Cu") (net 2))
 (segment (start 141.08484 90.861) (end 144.579 90.861) (width 0.2) (layer "B.Cu") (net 22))
 (segment (start 141.08484 53.409) (end 140.368 54.12584) (width 0.2) (layer "B.Cu") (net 22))
 (segment (start 147.922314 56.611) (end 144.28684 56.611) (width 0.2) (layer "B.Cu") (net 22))
 (segment (start 143.971 56.29516) (end 143.971 53.72484) (width 0.2) (layer "B.Cu") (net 22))
 (segment (start 163.690314 72.379) (end 147.922314 56.611) (width 0.2) (layer "B.Cu") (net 22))
 (segment (start 144.579 90.861) (end 146.18 89.26) (width 0.2) (layer "B.Cu") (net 22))
 (segment (start 144.28684 56.611) (end 143.971 56.29516) (width 0.2) (layer "B.Cu") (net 22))
 (segment (start 140.368 90.14416) (end 141.08484 90.861) (width 0.2) (layer "B.Cu") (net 22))
 (segment (start 140.368 54.12584) (end 140.368 90.14416) (width 0.2) (layer "B.Cu") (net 22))
 (segment (start 182.24 54.64) (end 181.429314 54.64) (width 0.2) (layer "B.Cu") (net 22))
 (segment (start 143.971 53.72484) (end 143.65516 53.409) (width 0.2) (layer "B.Cu") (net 22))
 (segment (start 181.429314 54.64) (end 163.690314 72.379) (width 0.2) (layer "B.Cu") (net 22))
 (segment (start 143.65516 53.409) (end 141.08484 53.409) (width 0.2) (layer "B.Cu") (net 22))
 (segment (start 195.720314 96.861) (end 196.541 96.040314) (width 0.2) (layer "F.Cu") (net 5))
 (segment (start 201.49 60.504816) (end 201.49 54.64) (width 0.2) (layer "F.Cu") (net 5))
 (segment (start 196.541 96.040314) (end 196.541 79.82253) (width 0.2) (layer "F.Cu") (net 5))
 (segment (start 193.26 68.734816) (end 201.49 60.504816) (width 0.2) (layer "F.Cu") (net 5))
 (segment (start 196.541 79.82253) (end 193.26 76.54153) (width 0.2) (layer "F.Cu") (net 5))
 (segment (start 150.491 100.421) (end 189.358314 100.421) (width 0.2) (layer "F.Cu") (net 5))
 (segment (start 193.26 76.54153) (end 193.26 68.734816) (width 0.2) (layer "F.Cu") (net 5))
 (segment (start 194.559686 96.861) (end 195.720314 96.861) (width 0.2) (layer "F.Cu") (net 5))
 (segment (start 193.739 96.040314) (end 194.559686 96.861) (width 0.2) (layer "F.Cu") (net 5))
 (segment (start 146.18 96.11) (end 150.491 100.421) (width 0.2) (layer "F.Cu") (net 5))
 (segment (start 189.358314 100.421) (end 193.739 96.040314) (width 0.2) (layer "F.Cu") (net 5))
 (segment (start 197.37153 102.96) (end 201.49 98.84153) (width 0.2) (layer "F.Cu") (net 18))
 (segment (start 201.49 98.84153) (end 201.49 92.92) (width 0.2) (layer "F.Cu") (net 18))
 (segment (start 146.18 102.96) (end 197.37153 102.96) (width 0.2) (layer "F.Cu") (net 18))
 (segment (start 175.86 95.53) (end 175.92 95.47) (width 0.2) (layer "F.Cu") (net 7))
 (segment (start 173.524 33.184) (end 173.524 45.02641) (width 0.2) (layer "F.Cu") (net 7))
 (segment (start 158.161 94.159) (end 156.79 95.53) (width 0.2) (layer "F.Cu") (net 7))
 (segment (start 168.056 45.884) (end 156.76 57.18) (width 0.2) (layer "F.Cu") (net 7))
 (segment (start 172.06 31.72) (end 173.524 33.184) (width 0.2) (layer "F.Cu") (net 7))
 (segment (start 173.524 45.02641) (end 172.66641 45.884) (width 0.2) (layer "F.Cu") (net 7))
 (segment (start 172.66641 45.884) (end 168.056 45.884) (width 0.2) (layer "F.Cu") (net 7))
 (segment (start 156.76 57.18) (end 158.161 58.581) (width 0.2) (layer "F.Cu") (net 7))
 (segment (start 158.161 58.581) (end 158.161 94.159) (width 0.2) (layer "F.Cu") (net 7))
 (segment (start 156.79 95.53) (end 175.86 95.53) (width 0.2) (layer "F.Cu") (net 7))
 (segment (start 156.76 82.2871) (end 156.76 76.32) (width 0.2) (layer "F.Cu") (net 8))
 (segment (start 144.579 56.19774) (end 140.368 60.40874) (width 0.2) (layer "F.Cu") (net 8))
 (segment (start 143.971 104.24516) (end 143.971 95.0761) (width 0.2) (layer "F.Cu") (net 8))
 (segment (start 144.579 54.346844) (end 144.579 56.19774) (width 0.2) (layer "F.Cu") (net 8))
 (segment (start 158.108844 40.817) (end 144.579 54.346844) (width 0.2) (layer "F.Cu") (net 8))
 (segment (start 172.50031 40.817) (end 158.108844 40.817) (width 0.2) (layer "F.Cu") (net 8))
 (segment (start 140.368 103.84416) (end 141.08484 104.561) (width 0.2) (layer "F.Cu") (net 8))
 (segment (start 140.368 60.40874) (end 140.368 103.84416) (width 0.2) (layer "F.Cu") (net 8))
 (segment (start 173.123 35.323) (end 173.123 40.19431) (width 0.2) (layer "F.Cu") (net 8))
 (segment (start 143.65516 104.561) (end 143.971 104.24516) (width 0.2) (layer "F.Cu") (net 8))
 (segment (start 141.08484 104.561) (end 143.65516 104.561) (width 0.2) (layer "F.Cu") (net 8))
 (segment (start 173.123 40.19431) (end 172.50031 40.817) (width 0.2) (layer "F.Cu") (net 8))
 (segment (start 143.971 95.0761) (end 156.76 82.2871) (width 0.2) (layer "F.Cu") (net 8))
 (segment (start 172.06 34.26) (end 173.123 35.323) (width 0.2) (layer "F.Cu") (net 8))
 (segment (start 169.953 76.32) (end 171.194 75.079) (width 0.2) (layer "B.Cu") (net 8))
 (segment (start 194.159 75.329) (end 195.23 76.4) (width 0.2) (layer "B.Cu") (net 8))
 (segment (start 179.35558 75.329) (end 194.159 75.329) (width 0.2) (layer "B.Cu") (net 8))
 (segment (start 171.194 75.079) (end 179.10558 75.079) (width 0.2) (layer "B.Cu") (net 8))
 (segment (start 179.10558 75.079) (end 179.35558 75.329) (width 0.2) (layer "B.Cu") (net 8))
 (segment (start 156.76 76.32) (end 169.953 76.32) (width 0.2) (layer "B.Cu") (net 8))
 (segment (start 194.71153 57.18) (end 195.14 57.18) (width 0.2) (layer "F.Cu") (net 6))
 (segment (start 195.14 57.18) (end 195.14 46.10237) (width 0.2) (layer "F.Cu") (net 6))
 (segment (start 195.14 57.18) (end 175.89 57.18) (width 0.2) (layer "F.Cu") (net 6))
 (segment (start 192.669 92.989) (end 192.669 59.22253) (width 0.2) (layer "F.Cu") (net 6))
 (segment (start 195.14 46.10237) (end 188.37763 39.34) (width 0.2) (layer "F.Cu") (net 6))
 (segment (start 195.14 95.46) (end 192.669 92.989) (width 0.2) (layer "F.Cu") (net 6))
 (segment (start 188.37763 39.34) (end 187.3 39.34) (width 0.2) (layer "F.Cu") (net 6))
 (segment (start 192.669 59.22253) (end 194.71153 57.18) (width 0.2) (layer "F.Cu") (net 6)))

